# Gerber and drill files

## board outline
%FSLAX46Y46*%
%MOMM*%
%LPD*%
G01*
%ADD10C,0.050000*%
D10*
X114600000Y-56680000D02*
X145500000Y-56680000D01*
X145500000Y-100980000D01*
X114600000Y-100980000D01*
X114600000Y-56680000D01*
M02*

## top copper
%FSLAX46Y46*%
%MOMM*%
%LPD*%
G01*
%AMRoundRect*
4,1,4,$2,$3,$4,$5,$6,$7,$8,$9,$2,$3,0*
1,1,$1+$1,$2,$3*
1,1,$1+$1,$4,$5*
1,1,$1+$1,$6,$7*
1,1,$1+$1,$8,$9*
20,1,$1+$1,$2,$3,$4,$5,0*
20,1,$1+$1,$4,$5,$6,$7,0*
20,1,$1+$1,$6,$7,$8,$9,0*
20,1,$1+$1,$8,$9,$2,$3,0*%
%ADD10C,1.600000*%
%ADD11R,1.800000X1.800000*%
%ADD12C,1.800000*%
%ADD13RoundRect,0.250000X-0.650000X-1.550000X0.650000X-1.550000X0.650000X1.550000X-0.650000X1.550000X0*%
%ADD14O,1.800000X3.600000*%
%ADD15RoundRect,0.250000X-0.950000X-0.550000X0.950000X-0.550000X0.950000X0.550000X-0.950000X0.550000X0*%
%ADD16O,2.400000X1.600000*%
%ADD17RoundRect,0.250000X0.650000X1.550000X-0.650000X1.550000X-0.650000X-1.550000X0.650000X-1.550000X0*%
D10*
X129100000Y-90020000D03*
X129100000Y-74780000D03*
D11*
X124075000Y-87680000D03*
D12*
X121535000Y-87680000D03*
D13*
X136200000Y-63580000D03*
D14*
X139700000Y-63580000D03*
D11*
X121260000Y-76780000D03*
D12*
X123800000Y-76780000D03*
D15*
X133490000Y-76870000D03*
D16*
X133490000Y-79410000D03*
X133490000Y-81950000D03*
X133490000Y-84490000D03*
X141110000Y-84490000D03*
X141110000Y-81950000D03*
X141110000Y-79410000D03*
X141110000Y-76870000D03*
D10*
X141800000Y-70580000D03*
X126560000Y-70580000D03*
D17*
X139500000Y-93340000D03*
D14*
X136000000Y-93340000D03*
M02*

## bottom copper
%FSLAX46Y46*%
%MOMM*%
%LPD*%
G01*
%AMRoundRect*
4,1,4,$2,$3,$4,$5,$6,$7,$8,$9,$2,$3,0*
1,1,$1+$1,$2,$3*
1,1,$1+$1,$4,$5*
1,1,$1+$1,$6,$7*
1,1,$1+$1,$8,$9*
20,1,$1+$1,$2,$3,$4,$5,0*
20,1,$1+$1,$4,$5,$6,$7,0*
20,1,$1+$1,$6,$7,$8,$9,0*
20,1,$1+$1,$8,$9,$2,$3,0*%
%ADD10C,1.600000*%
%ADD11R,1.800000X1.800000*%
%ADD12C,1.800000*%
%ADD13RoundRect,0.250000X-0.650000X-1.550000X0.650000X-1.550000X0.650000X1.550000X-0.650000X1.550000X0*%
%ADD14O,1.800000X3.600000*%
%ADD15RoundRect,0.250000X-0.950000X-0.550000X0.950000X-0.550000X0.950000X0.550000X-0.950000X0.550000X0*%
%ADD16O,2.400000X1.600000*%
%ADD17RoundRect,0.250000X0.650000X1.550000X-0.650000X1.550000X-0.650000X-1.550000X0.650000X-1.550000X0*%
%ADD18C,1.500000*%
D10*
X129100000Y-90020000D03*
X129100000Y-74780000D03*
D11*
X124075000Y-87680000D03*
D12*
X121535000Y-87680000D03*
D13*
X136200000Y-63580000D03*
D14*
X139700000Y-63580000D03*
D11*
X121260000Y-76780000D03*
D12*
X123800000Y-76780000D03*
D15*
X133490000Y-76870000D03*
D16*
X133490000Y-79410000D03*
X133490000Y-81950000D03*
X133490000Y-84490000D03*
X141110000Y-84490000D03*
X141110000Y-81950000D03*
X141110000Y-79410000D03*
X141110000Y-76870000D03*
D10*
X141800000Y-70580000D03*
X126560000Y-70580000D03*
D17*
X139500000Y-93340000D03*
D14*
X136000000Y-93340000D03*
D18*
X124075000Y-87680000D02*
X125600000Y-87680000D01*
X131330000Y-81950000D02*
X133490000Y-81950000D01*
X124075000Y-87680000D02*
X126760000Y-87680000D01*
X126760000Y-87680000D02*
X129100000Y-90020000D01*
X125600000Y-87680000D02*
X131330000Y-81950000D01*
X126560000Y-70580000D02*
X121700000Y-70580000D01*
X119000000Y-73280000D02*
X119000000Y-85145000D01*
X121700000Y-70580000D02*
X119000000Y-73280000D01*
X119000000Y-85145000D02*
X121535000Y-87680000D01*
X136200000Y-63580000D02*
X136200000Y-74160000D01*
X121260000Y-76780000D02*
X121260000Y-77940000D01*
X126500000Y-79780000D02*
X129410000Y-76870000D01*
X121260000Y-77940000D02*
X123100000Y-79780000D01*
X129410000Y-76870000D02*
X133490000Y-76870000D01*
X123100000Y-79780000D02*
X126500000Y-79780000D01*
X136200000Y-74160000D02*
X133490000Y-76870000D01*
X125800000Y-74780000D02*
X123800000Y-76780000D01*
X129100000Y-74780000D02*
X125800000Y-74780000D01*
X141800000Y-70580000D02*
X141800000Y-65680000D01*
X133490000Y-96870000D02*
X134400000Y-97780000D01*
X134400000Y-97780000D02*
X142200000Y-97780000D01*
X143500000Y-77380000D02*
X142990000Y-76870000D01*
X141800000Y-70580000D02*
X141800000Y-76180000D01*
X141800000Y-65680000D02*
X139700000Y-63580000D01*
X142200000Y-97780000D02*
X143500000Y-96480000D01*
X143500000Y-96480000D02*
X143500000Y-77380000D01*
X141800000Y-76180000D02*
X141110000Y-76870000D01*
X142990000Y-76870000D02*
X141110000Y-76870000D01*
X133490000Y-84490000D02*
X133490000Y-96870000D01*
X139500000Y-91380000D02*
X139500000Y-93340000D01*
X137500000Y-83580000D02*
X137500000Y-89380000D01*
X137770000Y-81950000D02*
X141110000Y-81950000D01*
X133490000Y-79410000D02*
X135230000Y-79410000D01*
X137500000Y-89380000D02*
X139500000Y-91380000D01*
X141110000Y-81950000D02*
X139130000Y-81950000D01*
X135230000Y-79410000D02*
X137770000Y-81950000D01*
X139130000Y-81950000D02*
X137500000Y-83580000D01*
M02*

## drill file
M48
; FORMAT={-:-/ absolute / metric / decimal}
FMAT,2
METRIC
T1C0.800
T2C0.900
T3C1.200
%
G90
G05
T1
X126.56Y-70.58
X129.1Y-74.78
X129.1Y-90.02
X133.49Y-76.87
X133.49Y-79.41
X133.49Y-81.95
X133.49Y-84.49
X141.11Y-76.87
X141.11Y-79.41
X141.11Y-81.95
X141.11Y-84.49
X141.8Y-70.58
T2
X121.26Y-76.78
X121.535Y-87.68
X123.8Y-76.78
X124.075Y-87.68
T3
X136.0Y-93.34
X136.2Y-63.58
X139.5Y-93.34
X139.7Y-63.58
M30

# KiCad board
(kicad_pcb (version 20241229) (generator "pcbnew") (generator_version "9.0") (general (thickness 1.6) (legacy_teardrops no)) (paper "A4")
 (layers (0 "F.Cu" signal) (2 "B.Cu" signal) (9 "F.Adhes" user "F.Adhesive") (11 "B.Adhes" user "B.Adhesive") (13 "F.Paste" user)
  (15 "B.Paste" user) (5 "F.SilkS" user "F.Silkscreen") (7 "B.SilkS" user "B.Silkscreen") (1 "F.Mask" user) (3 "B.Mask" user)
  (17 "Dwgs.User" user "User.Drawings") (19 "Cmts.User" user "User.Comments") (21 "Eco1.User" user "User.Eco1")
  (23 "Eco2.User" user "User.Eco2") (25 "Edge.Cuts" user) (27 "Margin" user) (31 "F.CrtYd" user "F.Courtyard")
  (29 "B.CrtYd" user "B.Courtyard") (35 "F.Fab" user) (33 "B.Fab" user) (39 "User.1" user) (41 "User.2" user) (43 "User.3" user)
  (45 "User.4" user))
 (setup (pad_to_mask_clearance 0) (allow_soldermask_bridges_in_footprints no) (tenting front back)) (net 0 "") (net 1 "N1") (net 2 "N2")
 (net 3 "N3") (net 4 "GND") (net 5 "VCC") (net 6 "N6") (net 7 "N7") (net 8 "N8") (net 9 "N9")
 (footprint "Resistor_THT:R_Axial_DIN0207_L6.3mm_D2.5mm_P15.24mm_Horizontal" (layer "F.Cu") (at 129.1 90.02 90)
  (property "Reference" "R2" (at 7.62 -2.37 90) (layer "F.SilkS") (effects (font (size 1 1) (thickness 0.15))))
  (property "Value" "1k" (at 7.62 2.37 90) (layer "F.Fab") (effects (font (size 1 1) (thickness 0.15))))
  (pad "1" thru_hole circle (at 0 0 90) (size 1.6 1.6) (drill 0.8) (layers "*.Cu" "*.Mask") (remove_unused_layers no) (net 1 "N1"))
  (pad "2" thru_hole circle (at 15.24 0 90) (size 1.6 1.6) (drill 0.8) (layers "*.Cu" "*.Mask") (remove_unused_layers no) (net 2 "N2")))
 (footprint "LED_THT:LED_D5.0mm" (layer "F.Cu") (at 124.075 87.68 180)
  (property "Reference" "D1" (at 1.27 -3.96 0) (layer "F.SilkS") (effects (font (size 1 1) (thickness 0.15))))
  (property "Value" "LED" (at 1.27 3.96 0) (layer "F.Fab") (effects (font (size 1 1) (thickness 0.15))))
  (pad "1" thru_hole rect (at 0 0 180) (size 1.8 1.8) (drill 0.9) (layers "*.Cu" "*.Mask") (remove_unused_layers no) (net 1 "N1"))
  (pad "2" thru_hole circle (at 2.54 0 180) (size 1.8 1.8) (drill 0.9) (layers "*.Cu" "*.Mask") (remove_unused_layers no) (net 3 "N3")))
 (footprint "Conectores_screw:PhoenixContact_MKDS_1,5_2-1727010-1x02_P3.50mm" (layer "F.Cu") (at 136.2 61.04)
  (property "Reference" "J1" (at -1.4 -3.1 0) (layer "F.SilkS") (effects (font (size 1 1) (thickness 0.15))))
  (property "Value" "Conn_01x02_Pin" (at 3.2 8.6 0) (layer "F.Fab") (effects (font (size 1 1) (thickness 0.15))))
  (pad "1" thru_hole roundrect (at 0 2.54) (size 1.8 3.6) (drill 1.2) (layers "*.Cu" "*.Mask") (remove_unused_layers no)
   (roundrect_rratio 0.138889) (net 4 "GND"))
  (pad "2" thru_hole oval (at 3.5 2.54) (size 1.8 3.6) (drill 1.2) (layers "*.Cu" "*.Mask") (remove_unused_layers no) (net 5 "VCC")))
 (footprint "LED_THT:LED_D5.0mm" (layer "F.Cu") (at 121.26 76.78)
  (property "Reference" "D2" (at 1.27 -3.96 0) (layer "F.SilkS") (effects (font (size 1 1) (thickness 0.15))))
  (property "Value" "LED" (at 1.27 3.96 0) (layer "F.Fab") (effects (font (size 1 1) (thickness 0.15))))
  (pad "1" thru_hole rect (at 0 0) (size 1.8 1.8) (drill 0.9) (layers "*.Cu" "*.Mask") (remove_unused_layers no) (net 4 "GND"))
  (pad "2" thru_hole circle (at 2.54 0) (size 1.8 1.8) (drill 0.9) (layers "*.Cu" "*.Mask") (remove_unused_layers no) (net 2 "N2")))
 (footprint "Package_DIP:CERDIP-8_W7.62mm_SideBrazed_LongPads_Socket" (layer "F.Cu") (at 133.49 76.87)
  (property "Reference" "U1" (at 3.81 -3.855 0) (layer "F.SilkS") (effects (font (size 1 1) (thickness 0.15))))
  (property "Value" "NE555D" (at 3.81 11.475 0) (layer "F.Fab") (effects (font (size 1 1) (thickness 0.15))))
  (pad "1" thru_hole roundrect (at 0 0) (size 2.4 1.6) (drill 0.8) (layers "*.Cu" "*.Mask") (remove_unused_layers no)
   (roundrect_rratio 0.15625) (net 4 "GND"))
  (pad "2" thru_hole oval (at 0 2.54) (size 2.4 1.6) (drill 0.8) (layers "*.Cu" "*.Mask") (remove_unused_layers no) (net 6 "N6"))
  (pad "3" thru_hole oval (at 0 5.08) (size 2.4 1.6) (drill 0.8) (layers "*.Cu" "*.Mask") (remove_unused_layers no) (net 1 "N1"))
  (pad "4" thru_hole oval (at 0 7.62) (size 2.4 1.6) (drill 0.8) (layers "*.Cu" "*.Mask") (remove_unused_layers no) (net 5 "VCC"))
  (pad "5" thru_hole oval (at 7.62 7.62) (size 2.4 1.6) (drill 0.8) (layers "*.Cu" "*.Mask") (remove_unused_layers no) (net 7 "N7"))
  (pad "6" thru_hole oval (at 7.62 5.08) (size 2.4 1.6) (drill 0.8) (layers "*.Cu" "*.Mask") (remove_unused_layers no) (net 6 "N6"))
  (pad "7" thru_hole oval (at 7.62 2.54) (size 2.4 1.6) (drill 0.8) (layers "*.Cu" "*.Mask") (remove_unused_layers no) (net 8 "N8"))
  (pad "8" thru_hole oval (at 7.62 0) (size 2.4 1.6) (drill 0.8) (layers "*.Cu" "*.Mask") (remove_unused_layers no) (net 5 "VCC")))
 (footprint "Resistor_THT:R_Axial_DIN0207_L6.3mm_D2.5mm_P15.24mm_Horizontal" (layer "F.Cu") (at 141.8 70.58 180)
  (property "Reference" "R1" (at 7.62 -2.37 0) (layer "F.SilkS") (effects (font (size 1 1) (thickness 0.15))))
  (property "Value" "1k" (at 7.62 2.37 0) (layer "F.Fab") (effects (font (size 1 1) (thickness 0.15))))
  (pad "1" thru_hole circle (at 0 0 180) (size 1.6 1.6) (drill 0.8) (layers "*.Cu" "*.Mask") (remove_unused_layers no) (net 5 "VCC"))
  (pad "2" thru_hole circle (at 15.24 0 180) (size 1.6 1.6) (drill 0.8) (layers "*.Cu" "*.Mask") (remove_unused_layers no) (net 3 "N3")))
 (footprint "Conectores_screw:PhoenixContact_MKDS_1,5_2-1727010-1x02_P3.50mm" (layer "F.Cu") (at 139.5 95.88 180)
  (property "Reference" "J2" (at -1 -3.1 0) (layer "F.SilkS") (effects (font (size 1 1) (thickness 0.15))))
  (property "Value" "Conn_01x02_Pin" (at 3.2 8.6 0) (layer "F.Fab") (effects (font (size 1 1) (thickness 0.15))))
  (pad "1" thru_hole roundrect (at 0 2.54 180) (size 1.8 3.6) (drill 1.2) (layers "*.Cu" "*.Mask") (remove_unused_layers no)
   (roundrect_rratio 0.138889) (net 6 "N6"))
  (pad "2" thru_hole oval (at 3.5 2.54 180) (size 1.8 3.6) (drill 1.2) (layers "*.Cu" "*.Mask") (remove_unused_layers no) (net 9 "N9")))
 (gr_rect (start 114.6 56.68) (end 145.5 100.98) (stroke (width 0.05) (type default)) (fill no) (layer "Edge.Cuts"))
 (segment (start 124.075 87.68) (end 125.6 87.68) (width 1.5) (layer "B.Cu") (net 1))
 (segment (start 131.33 81.95) (end 133.49 81.95) (width 1.5) (layer "B.Cu") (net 1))
 (segment (start 124.075 87.68) (end 126.76 87.68) (width 1.5) (layer "B.Cu") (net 1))
 (segment (start 126.76 87.68) (end 129.1 90.02) (width 1.5) (layer "B.Cu") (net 1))
 (segment (start 125.6 87.68) (end 131.33 81.95) (width 1.5) (layer "B.Cu") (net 1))
 (segment (start 126.56 70.58) (end 121.7 70.58) (width 1.5) (layer "B.Cu") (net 3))
 (segment (start 119 73.28) (end 119 85.145) (width 1.5) (layer "B.Cu") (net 3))
 (segment (start 121.7 70.58) (end 119 73.28) (width 1.5) (layer "B.Cu") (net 3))
 (segment (start 119 85.145) (end 121.535 87.68) (width 1.5) (layer "B.Cu") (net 3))
 (segment (start 136.2 63.58) (end 136.2 74.16) (width 1.5) (layer "B.Cu") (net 4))
 (segment (start 121.26 76.78) (end 121.26 77.94) (width 1.5) (layer "B.Cu") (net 4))
 (segment (start 126.5 79.78) (end 129.41 76.87) (width 1.5) (layer "B.Cu") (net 4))
 (segment (start 121.26 77.94) (end 123.1 79.78) (width 1.5) (layer "B.Cu") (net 4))
 (segment (start 129.41 76.87) (end 133.49 76.87) (width 1.5) (layer "B.Cu") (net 4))
 (segment (start 123.1 79.78) (end 126.5 79.78) (width 1.5) (layer "B.Cu") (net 4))
 (segment (start 136.2 74.16) (end 133.49 76.87) (width 1.5) (layer "B.Cu") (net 4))
 (segment (start 125.8 74.78) (end 123.8 76.78) (width 1.5) (layer "B.Cu") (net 2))
 (segment (start 129.1 74.78) (end 125.8 74.78) (width 1.5) (layer "B.Cu") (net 2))
 (segment (start 141.8 70.58) (end 141.8 65.68) (width 1.5) (layer "B.Cu") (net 5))
 (segment (start 133.49 96.87) (end 134.4 97.78) (width 1.5) (layer "B.Cu") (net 5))
 (segment (start 134.4 97.78) (end 142.2 97.78) (width 1.5) (layer "B.Cu") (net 5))
 (segment (start 143.5 77.38) (end 142.99 76.87) (width 1.5) (layer "B.Cu") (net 5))
 (segment (start 141.8 70.58) (end 141.8 76.18) (width 1.5) (layer "B.Cu") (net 5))
 (segment (start 141.8 65.68) (end 139.7 63.58) (width 1.5) (layer "B.Cu") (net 5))
 (segment (start 142.2 97.78) (end 143.5 96.48) (width 1.5) (layer "B.Cu") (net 5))
 (segment (start 143.5 96.48) (end 143.5 77.38) (width 1.5) (layer "B.Cu") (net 5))
 (segment (start 141.8 76.18) (end 141.11 76.87) (width 1.5) (layer "B.Cu") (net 5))
 (segment (start 142.99 76.87) (end 141.11 76.87) (width 1.5) (layer "B.Cu") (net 5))
 (segment (start 133.49 84.49) (end 133.49 96.87) (width 1.5) (layer "B.Cu") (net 5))
 (segment (start 139.5 91.38) (end 139.5 93.34) (width 1.5) (layer "B.Cu") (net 6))
 (segment (start 137.5 83.58) (end 137.5 89.38) (width 1.5) (layer "B.Cu") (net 6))
 (segment (start 137.77 81.95) (end 141.11 81.95) (width 1.5) (layer "B.Cu") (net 6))
 (segment (start 133.49 79.41) (end 135.23 79.41) (width 1.5) (layer "B.Cu") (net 6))
 (segment (start 137.5 89.38) (end 139.5 91.38) (width 1.5) (layer "B.Cu") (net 6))
 (segment (start 141.11 81.95) (end 139.13 81.95) (width 1.5) (layer "B.Cu") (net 6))
 (segment (start 135.23 79.41) (end 137.77 81.95) (width 1.5) (layer "B.Cu") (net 6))
 (segment (start 139.13 81.95) (end 137.5 83.58) (width 1.5) (layer "B.Cu") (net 6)))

